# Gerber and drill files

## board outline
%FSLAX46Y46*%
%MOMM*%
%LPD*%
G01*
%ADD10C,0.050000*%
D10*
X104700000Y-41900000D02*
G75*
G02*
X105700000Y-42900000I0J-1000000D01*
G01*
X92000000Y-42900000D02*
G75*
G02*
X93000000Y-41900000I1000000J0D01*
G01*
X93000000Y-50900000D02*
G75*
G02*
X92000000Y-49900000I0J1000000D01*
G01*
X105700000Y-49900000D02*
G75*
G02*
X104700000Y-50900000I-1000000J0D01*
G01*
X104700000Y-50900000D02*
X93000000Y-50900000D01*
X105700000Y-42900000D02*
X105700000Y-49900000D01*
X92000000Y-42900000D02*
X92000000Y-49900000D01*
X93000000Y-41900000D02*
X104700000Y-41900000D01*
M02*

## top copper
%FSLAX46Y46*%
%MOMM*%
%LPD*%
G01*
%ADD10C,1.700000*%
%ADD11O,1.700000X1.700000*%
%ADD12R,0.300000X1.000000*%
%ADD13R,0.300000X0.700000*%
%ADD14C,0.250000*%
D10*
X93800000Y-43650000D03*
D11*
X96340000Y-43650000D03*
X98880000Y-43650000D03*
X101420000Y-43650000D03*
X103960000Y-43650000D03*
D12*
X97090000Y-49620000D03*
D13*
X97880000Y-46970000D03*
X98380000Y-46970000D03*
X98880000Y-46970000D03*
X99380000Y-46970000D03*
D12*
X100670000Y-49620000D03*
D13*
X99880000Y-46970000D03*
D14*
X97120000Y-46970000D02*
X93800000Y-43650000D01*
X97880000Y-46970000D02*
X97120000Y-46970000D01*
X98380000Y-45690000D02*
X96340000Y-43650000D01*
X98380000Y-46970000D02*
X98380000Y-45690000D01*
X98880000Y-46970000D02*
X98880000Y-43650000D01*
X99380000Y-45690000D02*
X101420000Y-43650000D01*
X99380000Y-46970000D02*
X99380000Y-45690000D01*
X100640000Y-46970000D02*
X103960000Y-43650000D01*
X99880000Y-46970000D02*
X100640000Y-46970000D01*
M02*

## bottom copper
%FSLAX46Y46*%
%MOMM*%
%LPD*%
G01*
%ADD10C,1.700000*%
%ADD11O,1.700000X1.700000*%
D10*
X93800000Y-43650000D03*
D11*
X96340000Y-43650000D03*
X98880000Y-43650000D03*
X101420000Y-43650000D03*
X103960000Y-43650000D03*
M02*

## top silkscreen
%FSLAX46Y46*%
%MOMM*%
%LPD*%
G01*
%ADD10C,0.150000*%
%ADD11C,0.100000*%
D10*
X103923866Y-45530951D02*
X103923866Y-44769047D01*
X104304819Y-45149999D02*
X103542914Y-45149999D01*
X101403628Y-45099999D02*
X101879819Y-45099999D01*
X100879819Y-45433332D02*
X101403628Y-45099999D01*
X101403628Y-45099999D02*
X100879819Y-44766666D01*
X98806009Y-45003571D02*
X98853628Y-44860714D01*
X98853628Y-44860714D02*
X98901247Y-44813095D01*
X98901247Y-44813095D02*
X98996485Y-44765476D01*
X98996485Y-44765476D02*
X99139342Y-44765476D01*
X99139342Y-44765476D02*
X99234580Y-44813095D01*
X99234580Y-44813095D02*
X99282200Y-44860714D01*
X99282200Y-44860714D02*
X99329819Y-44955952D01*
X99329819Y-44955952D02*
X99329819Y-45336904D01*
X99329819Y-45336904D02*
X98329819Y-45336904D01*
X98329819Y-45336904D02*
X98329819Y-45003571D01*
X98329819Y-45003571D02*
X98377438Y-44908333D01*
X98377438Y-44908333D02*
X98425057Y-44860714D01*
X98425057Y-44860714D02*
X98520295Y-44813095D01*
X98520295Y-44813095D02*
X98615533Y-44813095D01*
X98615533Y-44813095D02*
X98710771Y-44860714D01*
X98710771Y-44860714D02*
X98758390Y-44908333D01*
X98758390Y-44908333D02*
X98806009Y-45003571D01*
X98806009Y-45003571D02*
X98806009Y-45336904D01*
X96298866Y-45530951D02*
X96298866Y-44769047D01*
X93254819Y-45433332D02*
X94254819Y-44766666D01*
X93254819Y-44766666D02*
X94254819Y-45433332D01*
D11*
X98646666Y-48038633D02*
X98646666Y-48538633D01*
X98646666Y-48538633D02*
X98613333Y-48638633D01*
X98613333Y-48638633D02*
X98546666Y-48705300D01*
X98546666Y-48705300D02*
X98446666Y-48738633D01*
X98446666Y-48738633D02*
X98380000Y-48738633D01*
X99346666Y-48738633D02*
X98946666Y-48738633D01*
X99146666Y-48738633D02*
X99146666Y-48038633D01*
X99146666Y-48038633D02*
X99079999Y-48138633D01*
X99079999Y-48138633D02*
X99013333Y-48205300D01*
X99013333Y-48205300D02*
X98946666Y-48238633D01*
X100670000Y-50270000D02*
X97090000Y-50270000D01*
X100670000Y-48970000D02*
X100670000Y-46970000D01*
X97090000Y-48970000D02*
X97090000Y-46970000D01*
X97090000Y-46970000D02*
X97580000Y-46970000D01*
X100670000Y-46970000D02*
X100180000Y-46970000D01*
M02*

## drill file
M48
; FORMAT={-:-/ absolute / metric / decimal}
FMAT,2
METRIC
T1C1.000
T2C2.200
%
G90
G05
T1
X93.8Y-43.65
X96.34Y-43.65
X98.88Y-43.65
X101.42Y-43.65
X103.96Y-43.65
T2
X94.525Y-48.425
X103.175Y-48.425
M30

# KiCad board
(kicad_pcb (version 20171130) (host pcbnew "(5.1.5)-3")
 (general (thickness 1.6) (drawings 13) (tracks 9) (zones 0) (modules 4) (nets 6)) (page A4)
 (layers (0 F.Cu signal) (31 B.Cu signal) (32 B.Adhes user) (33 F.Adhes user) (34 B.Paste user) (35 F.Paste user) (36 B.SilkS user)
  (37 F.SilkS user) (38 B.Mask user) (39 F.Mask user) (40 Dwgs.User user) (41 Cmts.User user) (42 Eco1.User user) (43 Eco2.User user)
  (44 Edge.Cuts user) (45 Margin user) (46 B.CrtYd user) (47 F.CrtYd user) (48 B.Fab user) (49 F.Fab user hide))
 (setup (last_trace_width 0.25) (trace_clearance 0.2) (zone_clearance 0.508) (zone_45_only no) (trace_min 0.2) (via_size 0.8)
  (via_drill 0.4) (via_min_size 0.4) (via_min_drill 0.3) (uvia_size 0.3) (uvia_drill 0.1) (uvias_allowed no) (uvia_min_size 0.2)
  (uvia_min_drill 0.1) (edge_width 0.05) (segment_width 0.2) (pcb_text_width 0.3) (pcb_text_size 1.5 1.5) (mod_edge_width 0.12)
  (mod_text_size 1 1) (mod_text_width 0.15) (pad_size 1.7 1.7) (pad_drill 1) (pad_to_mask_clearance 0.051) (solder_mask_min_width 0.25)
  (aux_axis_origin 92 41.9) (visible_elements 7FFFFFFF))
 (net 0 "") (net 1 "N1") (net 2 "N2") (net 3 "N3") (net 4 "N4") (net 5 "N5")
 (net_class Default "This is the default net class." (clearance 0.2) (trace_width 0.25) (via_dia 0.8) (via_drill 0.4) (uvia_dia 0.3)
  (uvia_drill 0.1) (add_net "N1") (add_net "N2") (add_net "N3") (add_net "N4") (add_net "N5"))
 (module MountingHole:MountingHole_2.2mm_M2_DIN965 (layer F.Cu) (at 94.525 48.425)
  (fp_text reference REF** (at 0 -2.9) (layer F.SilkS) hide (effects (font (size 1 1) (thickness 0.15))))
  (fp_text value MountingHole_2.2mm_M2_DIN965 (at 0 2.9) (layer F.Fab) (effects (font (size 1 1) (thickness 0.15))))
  (pad 1 np_thru_hole circle (at 0 0) (size 2.2 2.2) (drill 2.2) (layers *.Cu *.Mask)))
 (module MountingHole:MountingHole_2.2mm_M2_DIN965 (layer F.Cu) (at 103.175 48.425)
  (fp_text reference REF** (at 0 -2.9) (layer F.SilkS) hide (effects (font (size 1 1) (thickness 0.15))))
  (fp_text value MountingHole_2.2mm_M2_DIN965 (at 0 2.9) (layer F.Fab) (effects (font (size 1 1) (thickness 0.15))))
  (pad 1 np_thru_hole circle (at 0 0) (size 2.2 2.2) (drill 2.2) (layers *.Cu *.Mask)))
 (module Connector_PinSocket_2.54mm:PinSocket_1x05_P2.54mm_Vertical (layer F.Cu) (at 92 41.9 90)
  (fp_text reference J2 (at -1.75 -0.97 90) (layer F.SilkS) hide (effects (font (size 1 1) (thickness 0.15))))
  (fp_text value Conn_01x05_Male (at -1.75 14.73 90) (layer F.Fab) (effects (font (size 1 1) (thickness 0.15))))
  (pad 1 thru_hole circle (at -1.75 1.8 90) (size 1.7 1.7) (drill 1) (layers *.Cu *.Mask) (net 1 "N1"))
  (pad 2 thru_hole oval (at -1.75 4.34 90) (size 1.7 1.7) (drill 1) (layers *.Cu *.Mask) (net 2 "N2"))
  (pad 3 thru_hole oval (at -1.75 6.88 90) (size 1.7 1.7) (drill 1) (layers *.Cu *.Mask) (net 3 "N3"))
  (pad 4 thru_hole oval (at -1.75 9.42 90) (size 1.7 1.7) (drill 1) (layers *.Cu *.Mask) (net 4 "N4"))
  (pad 5 thru_hole oval (at -1.75 11.96 90) (size 1.7 1.7) (drill 1) (layers *.Cu *.Mask) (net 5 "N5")))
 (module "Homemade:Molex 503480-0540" (layer F.Cu) (at 98.88 48.42)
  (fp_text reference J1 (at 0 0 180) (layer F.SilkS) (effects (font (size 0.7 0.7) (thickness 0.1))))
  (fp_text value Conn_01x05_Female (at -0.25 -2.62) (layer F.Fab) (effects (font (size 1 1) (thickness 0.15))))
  (fp_line (start 1.79 1.85) (end -1.79 1.85) (layer F.SilkS) (width 0.1))
  (fp_line (start 1.79 0.55) (end 1.79 -1.45) (layer F.SilkS) (width 0.1))
  (fp_line (start -1.79 0.55) (end -1.79 -1.45) (layer F.SilkS) (width 0.1))
  (fp_line (start -1.79 -1.45) (end -1.3 -1.45) (layer F.SilkS) (width 0.1))
  (fp_line (start 1.79 -1.45) (end 1.3 -1.45) (layer F.SilkS) (width 0.1))
  (pad 6 smd rect (at -1.79 1.2) (size 0.3 1) (layers F.Cu F.Paste F.Mask))
  (pad 1 smd rect (at -1 -1.45) (size 0.3 0.7) (layers F.Cu F.Paste F.Mask) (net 1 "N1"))
  (pad 2 smd rect (at -0.5 -1.45) (size 0.3 0.7) (layers F.Cu F.Paste F.Mask) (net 2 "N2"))
  (pad 3 smd rect (at 0 -1.45) (size 0.3 0.7) (layers F.Cu F.Paste F.Mask) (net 3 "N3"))
  (pad 4 smd rect (at 0.5 -1.45) (size 0.3 0.7) (layers F.Cu F.Paste F.Mask) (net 4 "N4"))
  (pad 7 smd rect (at 1.79 1.2) (size 0.3 1) (layers F.Cu F.Paste F.Mask))
  (pad 5 smd rect (at 1 -1.45) (size 0.3 0.7) (layers F.Cu F.Paste F.Mask) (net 5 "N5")))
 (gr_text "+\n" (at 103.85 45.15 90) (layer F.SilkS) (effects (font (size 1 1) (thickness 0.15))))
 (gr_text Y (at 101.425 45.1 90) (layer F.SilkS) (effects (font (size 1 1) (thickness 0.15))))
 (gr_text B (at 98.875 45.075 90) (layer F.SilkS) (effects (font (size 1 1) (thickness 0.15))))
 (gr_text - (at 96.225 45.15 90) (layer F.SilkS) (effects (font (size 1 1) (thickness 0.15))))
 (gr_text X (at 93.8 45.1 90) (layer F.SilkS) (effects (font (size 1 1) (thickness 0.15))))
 (gr_arc (start 104.7 42.9) (end 105.7 42.9) (angle -90) (layer Edge.Cuts) (width 0.05))
 (gr_arc (start 93 42.9) (end 93 41.9) (angle -90) (layer Edge.Cuts) (width 0.05))
 (gr_arc (start 93 49.9) (end 92 49.9) (angle -90) (layer Edge.Cuts) (width 0.05))
 (gr_arc (start 104.7 49.9) (end 104.7 50.9) (angle -90) (layer Edge.Cuts) (width 0.05))
 (gr_line (start 104.7 50.9) (end 93 50.9) (layer Edge.Cuts) (width 0.05))
 (gr_line (start 105.7 42.9) (end 105.7 49.9) (layer Edge.Cuts) (width 0.05))
 (gr_line (start 92 42.9) (end 92 49.9) (layer Edge.Cuts) (width 0.05))
 (gr_line (start 93 41.9) (end 104.7 41.9) (layer Edge.Cuts) (width 0.05))
 (segment (start 97.12 46.97) (end 93.8 43.65) (width 0.25) (layer F.Cu) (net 1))
 (segment (start 97.88 46.97) (end 97.12 46.97) (width 0.25) (layer F.Cu) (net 1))
 (segment (start 98.38 45.69) (end 96.34 43.65) (width 0.25) (layer F.Cu) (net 2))
 (segment (start 98.38 46.97) (end 98.38 45.69) (width 0.25) (layer F.Cu) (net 2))
 (segment (start 98.88 46.97) (end 98.88 43.65) (width 0.25) (layer F.Cu) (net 3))
 (segment (start 99.38 45.69) (end 101.42 43.65) (width 0.25) (layer F.Cu) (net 4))
 (segment (start 99.38 46.97) (end 99.38 45.69) (width 0.25) (layer F.Cu) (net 4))
 (segment (start 100.64 46.97) (end 103.96 43.65) (width 0.25) (layer F.Cu) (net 5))
 (segment (start 99.88 46.97) (end 100.64 46.97) (width 0.25) (layer F.Cu) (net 5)))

